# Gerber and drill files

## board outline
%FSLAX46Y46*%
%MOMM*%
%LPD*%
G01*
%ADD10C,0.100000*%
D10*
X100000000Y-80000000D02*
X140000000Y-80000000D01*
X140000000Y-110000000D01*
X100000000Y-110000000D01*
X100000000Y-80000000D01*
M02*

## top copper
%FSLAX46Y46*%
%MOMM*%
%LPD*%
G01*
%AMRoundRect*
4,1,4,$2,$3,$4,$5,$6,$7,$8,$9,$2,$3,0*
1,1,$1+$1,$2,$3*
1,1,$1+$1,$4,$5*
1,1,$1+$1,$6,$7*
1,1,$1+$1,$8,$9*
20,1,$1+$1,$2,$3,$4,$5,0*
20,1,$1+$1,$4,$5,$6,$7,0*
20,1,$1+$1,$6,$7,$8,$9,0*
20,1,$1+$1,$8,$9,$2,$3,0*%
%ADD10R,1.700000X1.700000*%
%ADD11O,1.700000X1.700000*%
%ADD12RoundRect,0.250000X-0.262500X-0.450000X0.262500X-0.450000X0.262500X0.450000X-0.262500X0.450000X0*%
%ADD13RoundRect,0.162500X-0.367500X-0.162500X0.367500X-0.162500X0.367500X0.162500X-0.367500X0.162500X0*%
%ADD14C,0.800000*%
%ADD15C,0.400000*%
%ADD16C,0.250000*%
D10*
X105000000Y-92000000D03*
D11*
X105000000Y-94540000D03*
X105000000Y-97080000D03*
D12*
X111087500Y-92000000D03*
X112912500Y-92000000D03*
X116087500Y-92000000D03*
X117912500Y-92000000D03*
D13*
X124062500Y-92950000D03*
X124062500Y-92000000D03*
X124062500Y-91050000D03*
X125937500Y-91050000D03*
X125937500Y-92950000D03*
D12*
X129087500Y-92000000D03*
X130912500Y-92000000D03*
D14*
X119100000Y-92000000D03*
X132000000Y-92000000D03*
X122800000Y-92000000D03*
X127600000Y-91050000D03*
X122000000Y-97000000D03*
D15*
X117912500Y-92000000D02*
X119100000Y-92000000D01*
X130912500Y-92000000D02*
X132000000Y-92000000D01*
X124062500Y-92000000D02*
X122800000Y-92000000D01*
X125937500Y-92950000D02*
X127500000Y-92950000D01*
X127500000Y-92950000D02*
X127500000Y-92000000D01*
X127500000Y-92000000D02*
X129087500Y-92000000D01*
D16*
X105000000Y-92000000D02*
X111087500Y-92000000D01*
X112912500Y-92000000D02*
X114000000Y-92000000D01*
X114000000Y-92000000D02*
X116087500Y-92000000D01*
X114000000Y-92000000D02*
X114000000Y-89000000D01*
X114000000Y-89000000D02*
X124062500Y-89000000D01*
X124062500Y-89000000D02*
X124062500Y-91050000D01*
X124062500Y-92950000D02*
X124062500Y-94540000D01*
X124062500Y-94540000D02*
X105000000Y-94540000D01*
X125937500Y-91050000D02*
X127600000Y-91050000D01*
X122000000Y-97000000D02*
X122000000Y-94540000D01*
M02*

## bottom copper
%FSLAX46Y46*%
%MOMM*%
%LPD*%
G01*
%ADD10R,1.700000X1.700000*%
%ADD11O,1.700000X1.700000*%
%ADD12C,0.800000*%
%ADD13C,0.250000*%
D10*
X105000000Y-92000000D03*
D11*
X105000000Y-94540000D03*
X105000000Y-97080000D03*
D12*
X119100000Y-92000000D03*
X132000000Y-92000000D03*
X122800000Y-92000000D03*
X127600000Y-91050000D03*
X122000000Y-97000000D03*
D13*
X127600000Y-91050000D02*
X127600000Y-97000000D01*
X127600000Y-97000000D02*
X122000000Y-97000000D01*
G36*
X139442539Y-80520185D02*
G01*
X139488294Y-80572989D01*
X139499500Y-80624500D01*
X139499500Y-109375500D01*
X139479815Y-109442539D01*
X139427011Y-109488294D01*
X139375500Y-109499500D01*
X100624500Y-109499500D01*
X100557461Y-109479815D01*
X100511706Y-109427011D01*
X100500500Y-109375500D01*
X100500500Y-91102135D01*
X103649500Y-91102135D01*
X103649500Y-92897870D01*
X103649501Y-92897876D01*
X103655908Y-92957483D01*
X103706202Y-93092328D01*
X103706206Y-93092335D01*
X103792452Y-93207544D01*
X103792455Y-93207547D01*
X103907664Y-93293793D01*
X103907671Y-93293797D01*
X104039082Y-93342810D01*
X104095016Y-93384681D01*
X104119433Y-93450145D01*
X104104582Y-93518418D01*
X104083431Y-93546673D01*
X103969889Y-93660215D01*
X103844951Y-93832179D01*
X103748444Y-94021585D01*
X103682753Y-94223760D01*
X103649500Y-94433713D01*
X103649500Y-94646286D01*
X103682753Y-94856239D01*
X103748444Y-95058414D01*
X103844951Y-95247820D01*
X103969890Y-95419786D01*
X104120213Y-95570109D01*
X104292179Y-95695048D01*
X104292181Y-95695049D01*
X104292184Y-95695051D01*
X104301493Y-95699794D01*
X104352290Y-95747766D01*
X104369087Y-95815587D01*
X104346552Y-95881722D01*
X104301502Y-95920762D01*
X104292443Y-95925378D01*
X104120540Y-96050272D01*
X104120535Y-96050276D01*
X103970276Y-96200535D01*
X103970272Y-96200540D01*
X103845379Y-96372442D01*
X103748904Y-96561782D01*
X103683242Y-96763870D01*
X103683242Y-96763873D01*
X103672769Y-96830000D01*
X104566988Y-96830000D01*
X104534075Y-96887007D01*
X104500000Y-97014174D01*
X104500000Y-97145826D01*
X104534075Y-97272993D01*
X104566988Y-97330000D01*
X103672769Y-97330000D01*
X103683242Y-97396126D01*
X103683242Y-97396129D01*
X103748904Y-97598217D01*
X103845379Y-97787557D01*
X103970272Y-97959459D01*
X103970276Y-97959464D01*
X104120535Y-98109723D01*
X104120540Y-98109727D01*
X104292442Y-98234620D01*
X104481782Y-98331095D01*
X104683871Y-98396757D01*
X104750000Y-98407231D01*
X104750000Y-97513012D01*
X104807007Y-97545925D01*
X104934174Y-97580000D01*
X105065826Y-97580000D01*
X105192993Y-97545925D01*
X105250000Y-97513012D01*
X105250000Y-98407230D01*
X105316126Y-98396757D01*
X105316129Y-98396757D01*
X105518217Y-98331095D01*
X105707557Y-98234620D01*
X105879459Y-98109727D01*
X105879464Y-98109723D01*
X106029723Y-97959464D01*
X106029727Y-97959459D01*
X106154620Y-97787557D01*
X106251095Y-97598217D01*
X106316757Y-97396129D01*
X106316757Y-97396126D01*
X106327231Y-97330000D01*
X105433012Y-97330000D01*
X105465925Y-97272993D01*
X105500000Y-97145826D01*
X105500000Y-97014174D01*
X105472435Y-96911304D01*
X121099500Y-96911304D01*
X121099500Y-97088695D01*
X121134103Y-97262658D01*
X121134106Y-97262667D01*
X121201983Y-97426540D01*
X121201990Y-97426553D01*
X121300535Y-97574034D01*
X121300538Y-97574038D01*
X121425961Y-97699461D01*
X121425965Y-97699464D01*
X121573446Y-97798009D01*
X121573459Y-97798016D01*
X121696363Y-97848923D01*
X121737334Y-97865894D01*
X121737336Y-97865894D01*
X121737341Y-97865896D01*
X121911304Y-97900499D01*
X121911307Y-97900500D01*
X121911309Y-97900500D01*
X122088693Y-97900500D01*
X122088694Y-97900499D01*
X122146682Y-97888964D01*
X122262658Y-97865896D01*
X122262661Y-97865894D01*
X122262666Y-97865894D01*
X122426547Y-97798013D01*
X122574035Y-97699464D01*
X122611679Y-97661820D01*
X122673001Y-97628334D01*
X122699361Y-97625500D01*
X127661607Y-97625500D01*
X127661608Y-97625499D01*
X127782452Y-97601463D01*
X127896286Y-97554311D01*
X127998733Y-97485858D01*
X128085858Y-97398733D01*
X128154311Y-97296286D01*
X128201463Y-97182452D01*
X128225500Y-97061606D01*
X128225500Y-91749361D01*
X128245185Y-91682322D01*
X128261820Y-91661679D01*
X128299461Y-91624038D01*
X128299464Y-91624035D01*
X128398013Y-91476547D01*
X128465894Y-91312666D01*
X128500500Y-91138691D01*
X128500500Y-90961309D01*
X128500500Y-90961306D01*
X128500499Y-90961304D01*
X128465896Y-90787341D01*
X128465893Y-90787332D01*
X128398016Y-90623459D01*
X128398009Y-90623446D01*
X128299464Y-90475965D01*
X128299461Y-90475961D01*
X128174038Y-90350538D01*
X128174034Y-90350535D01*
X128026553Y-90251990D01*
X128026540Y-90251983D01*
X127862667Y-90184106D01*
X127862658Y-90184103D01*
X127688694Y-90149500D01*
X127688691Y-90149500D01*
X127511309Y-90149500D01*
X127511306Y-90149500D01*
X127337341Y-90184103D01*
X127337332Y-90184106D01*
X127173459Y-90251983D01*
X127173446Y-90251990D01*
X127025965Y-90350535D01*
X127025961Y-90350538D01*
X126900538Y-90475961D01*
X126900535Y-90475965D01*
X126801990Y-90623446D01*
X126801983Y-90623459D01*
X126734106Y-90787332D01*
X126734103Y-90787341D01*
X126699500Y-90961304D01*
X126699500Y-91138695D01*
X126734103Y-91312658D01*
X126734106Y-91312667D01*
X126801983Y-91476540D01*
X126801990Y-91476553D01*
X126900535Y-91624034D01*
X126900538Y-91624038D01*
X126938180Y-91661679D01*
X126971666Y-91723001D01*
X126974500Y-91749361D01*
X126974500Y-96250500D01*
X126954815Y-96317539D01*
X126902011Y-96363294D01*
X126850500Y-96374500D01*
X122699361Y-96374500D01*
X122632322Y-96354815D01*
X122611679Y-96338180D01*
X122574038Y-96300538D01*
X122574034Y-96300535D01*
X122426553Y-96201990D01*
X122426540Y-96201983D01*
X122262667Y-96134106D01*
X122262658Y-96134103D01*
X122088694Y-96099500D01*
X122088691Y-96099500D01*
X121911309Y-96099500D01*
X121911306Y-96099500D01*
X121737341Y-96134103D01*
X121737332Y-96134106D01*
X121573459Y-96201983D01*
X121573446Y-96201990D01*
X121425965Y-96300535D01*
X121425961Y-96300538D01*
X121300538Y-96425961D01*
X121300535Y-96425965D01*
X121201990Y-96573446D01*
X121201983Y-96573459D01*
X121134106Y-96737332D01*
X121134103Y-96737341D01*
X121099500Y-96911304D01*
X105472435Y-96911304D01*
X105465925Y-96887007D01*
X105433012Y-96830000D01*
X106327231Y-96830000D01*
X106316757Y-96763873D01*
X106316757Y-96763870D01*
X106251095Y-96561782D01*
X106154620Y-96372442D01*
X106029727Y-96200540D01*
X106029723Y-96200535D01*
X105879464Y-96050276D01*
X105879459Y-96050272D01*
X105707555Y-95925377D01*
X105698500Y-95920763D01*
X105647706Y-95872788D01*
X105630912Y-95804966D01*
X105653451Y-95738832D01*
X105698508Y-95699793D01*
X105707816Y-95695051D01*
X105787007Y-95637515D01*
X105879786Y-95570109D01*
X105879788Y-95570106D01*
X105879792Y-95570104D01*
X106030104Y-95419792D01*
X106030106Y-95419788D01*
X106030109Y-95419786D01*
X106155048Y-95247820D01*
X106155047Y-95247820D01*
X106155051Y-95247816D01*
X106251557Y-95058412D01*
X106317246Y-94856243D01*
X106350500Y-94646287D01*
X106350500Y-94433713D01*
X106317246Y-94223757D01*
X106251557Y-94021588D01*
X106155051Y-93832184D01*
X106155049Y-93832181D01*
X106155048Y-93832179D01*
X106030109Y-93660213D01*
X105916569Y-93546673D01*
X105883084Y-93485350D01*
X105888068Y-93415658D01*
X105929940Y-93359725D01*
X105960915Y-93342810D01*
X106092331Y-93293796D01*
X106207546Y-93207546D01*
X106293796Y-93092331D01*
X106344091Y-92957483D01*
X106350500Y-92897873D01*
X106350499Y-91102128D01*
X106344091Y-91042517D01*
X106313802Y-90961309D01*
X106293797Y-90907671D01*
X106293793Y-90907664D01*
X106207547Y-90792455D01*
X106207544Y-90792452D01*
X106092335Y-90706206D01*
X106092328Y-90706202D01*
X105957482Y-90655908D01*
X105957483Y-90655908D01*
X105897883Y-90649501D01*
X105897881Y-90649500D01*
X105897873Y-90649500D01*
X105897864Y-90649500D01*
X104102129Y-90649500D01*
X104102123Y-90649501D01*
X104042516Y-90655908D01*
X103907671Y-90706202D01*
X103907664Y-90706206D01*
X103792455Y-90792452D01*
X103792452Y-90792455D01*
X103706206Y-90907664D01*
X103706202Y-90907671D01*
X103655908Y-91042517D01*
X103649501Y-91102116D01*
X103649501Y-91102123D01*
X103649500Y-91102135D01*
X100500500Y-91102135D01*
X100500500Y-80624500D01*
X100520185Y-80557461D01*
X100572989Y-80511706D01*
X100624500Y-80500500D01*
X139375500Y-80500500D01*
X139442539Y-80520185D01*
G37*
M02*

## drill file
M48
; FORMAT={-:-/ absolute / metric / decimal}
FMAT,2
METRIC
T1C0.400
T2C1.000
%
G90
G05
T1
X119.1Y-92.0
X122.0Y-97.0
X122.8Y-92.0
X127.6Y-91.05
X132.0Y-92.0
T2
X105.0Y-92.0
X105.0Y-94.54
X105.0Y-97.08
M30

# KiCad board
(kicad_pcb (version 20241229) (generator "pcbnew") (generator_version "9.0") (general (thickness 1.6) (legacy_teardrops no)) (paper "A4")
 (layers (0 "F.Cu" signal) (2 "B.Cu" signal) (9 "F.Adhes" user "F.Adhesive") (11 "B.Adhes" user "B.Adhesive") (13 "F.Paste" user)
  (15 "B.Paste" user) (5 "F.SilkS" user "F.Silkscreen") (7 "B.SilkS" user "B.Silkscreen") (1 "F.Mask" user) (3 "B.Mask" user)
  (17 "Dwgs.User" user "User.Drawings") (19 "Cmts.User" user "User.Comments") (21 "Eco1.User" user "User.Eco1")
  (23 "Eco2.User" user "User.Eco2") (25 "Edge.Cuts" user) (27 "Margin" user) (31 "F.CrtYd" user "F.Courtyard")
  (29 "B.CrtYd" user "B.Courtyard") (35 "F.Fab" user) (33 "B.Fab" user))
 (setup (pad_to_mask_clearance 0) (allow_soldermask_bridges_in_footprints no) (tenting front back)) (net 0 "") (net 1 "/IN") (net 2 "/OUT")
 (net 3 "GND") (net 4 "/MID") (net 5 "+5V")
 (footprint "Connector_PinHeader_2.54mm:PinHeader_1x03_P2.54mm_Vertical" (layer "F.Cu") (at 105 92)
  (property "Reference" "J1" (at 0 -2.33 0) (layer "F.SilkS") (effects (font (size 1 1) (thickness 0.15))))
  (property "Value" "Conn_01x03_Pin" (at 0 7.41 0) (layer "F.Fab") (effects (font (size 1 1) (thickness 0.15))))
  (pad "1" thru_hole rect (at 0 0) (size 1.7 1.7) (drill 1) (layers "*.Cu" "*.Mask") (remove_unused_layers no) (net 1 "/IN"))
  (pad "2" thru_hole oval (at 0 2.54) (size 1.7 1.7) (drill 1) (layers "*.Cu" "*.Mask") (remove_unused_layers no) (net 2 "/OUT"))
  (pad "3" thru_hole oval (at 0 5.08) (size 1.7 1.7) (drill 1) (layers "*.Cu" "*.Mask") (remove_unused_layers no) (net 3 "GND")))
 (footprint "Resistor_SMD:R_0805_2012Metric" (layer "F.Cu") (at 112 92)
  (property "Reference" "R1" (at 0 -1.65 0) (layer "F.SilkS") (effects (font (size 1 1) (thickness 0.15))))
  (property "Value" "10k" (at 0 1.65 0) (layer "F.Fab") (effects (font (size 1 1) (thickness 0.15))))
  (pad "1" smd roundrect (at -0.9125 0) (size 1.025 1.4) (layers "F.Cu" "F.Mask" "F.Paste") (roundrect_rratio 0.243902) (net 1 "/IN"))
  (pad "2" smd roundrect (at 0.9125 0) (size 1.025 1.4) (layers "F.Cu" "F.Mask" "F.Paste") (roundrect_rratio 0.243902) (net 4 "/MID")))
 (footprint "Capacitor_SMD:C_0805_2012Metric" (layer "F.Cu") (at 117 92)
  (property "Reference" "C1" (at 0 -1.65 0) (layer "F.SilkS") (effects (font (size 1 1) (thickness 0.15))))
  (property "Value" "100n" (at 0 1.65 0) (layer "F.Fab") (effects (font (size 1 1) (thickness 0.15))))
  (pad "1" smd roundrect (at -0.9125 0) (size 1.025 1.4) (layers "F.Cu" "F.Mask" "F.Paste") (roundrect_rratio 0.243902) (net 4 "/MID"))
  (pad "2" smd roundrect (at 0.9125 0) (size 1.025 1.4) (layers "F.Cu" "F.Mask" "F.Paste") (roundrect_rratio 0.243902) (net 3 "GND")))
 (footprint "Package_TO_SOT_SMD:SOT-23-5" (layer "F.Cu") (at 125 92)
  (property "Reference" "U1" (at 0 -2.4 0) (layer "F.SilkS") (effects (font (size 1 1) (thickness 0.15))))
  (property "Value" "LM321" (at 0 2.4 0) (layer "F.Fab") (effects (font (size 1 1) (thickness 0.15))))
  (pad "1" smd roundrect (at -0.9375 0.95) (size 1.06 0.65) (layers "F.Cu" "F.Mask" "F.Paste") (roundrect_rratio 0.25) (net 2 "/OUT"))
  (pad "2" smd roundrect (at -0.9375 0) (size 1.06 0.65) (layers "F.Cu" "F.Mask" "F.Paste") (roundrect_rratio 0.25) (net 3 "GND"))
  (pad "3" smd roundrect (at -0.9375 -0.95) (size 1.06 0.65) (layers "F.Cu" "F.Mask" "F.Paste") (roundrect_rratio 0.25) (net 4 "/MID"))
  (pad "4" smd roundrect (at 0.9375 -0.95) (size 1.06 0.65) (layers "F.Cu" "F.Mask" "F.Paste") (roundrect_rratio 0.25) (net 2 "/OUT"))
  (pad "5" smd roundrect (at 0.9375 0.95) (size 1.06 0.65) (layers "F.Cu" "F.Mask" "F.Paste") (roundrect_rratio 0.25) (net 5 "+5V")))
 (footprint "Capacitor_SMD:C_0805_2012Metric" (layer "F.Cu") (at 130 92)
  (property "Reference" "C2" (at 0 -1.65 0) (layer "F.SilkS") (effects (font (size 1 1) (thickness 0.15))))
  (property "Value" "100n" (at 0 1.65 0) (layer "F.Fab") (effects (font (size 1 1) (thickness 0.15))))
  (pad "1" smd roundrect (at -0.9125 0) (size 1.025 1.4) (layers "F.Cu" "F.Mask" "F.Paste") (roundrect_rratio 0.243902) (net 5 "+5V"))
  (pad "2" smd roundrect (at 0.9125 0) (size 1.025 1.4) (layers "F.Cu" "F.Mask" "F.Paste") (roundrect_rratio 0.243902) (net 3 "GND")))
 (gr_rect (start 100 80) (end 140 110) (stroke (width 0.1) (type default)) (fill no) (layer "Edge.Cuts"))
 (segment (start 117.9125 92) (end 119.1 92) (width 0.4) (layer "F.Cu") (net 3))
 (segment (start 130.9125 92) (end 132 92) (width 0.4) (layer "F.Cu") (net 3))
 (segment (start 124.0625 92) (end 122.8 92) (width 0.4) (layer "F.Cu") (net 3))
 (via (at 119.1 92) (size 0.8) (drill 0.4) (layers "F.Cu" "B.Cu") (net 3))
 (via (at 132 92) (size 0.8) (drill 0.4) (layers "F.Cu" "B.Cu") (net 3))
 (via (at 122.8 92) (size 0.8) (drill 0.4) (layers "F.Cu" "B.Cu") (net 3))
 (segment (start 125.9375 92.95) (end 127.5 92.95) (width 0.4) (layer "F.Cu") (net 5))
 (segment (start 127.5 92.95) (end 127.5 92) (width 0.4) (layer "F.Cu") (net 5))
 (segment (start 127.5 92) (end 129.0875 92) (width 0.4) (layer "F.Cu") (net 5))
 (segment (start 105 92) (end 111.0875 92) (width 0.25) (layer "F.Cu") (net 1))
 (segment (start 112.9125 92) (end 114 92) (width 0.25) (layer "F.Cu") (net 4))
 (segment (start 114 92) (end 116.0875 92) (width 0.25) (layer "F.Cu") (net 4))
 (segment (start 114 92) (end 114 89) (width 0.25) (layer "F.Cu") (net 4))
 (segment (start 114 89) (end 124.0625 89) (width 0.25) (layer "F.Cu") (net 4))
 (segment (start 124.0625 89) (end 124.0625 91.05) (width 0.25) (layer "F.Cu") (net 4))
 (segment (start 124.0625 92.95) (end 124.0625 94.54) (width 0.25) (layer "F.Cu") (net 2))
 (segment (start 124.0625 94.54) (end 105 94.54) (width 0.25) (layer "F.Cu") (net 2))
 (segment (start 125.9375 91.05) (end 127.6 91.05) (width 0.25) (layer "F.Cu") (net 2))
 (segment (start 122 97) (end 122 94.54) (width 0.25) (layer "F.Cu") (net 2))
 (via (at 127.6 91.05) (size 0.8) (drill 0.4) (layers "F.Cu" "B.Cu") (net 2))
 (via (at 122 97) (size 0.8) (drill 0.4) (layers "F.Cu" "B.Cu") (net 2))
 (segment (start 127.6 91.05) (end 127.6 97) (width 0.25) (layer "B.Cu") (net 2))
 (segment (start 127.6 97) (end 122 97) (width 0.25) (layer "B.Cu") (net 2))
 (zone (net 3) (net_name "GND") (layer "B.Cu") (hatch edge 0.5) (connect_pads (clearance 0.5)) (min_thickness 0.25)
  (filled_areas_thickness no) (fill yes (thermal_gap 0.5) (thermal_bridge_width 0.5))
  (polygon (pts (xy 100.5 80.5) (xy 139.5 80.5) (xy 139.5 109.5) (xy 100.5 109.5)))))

